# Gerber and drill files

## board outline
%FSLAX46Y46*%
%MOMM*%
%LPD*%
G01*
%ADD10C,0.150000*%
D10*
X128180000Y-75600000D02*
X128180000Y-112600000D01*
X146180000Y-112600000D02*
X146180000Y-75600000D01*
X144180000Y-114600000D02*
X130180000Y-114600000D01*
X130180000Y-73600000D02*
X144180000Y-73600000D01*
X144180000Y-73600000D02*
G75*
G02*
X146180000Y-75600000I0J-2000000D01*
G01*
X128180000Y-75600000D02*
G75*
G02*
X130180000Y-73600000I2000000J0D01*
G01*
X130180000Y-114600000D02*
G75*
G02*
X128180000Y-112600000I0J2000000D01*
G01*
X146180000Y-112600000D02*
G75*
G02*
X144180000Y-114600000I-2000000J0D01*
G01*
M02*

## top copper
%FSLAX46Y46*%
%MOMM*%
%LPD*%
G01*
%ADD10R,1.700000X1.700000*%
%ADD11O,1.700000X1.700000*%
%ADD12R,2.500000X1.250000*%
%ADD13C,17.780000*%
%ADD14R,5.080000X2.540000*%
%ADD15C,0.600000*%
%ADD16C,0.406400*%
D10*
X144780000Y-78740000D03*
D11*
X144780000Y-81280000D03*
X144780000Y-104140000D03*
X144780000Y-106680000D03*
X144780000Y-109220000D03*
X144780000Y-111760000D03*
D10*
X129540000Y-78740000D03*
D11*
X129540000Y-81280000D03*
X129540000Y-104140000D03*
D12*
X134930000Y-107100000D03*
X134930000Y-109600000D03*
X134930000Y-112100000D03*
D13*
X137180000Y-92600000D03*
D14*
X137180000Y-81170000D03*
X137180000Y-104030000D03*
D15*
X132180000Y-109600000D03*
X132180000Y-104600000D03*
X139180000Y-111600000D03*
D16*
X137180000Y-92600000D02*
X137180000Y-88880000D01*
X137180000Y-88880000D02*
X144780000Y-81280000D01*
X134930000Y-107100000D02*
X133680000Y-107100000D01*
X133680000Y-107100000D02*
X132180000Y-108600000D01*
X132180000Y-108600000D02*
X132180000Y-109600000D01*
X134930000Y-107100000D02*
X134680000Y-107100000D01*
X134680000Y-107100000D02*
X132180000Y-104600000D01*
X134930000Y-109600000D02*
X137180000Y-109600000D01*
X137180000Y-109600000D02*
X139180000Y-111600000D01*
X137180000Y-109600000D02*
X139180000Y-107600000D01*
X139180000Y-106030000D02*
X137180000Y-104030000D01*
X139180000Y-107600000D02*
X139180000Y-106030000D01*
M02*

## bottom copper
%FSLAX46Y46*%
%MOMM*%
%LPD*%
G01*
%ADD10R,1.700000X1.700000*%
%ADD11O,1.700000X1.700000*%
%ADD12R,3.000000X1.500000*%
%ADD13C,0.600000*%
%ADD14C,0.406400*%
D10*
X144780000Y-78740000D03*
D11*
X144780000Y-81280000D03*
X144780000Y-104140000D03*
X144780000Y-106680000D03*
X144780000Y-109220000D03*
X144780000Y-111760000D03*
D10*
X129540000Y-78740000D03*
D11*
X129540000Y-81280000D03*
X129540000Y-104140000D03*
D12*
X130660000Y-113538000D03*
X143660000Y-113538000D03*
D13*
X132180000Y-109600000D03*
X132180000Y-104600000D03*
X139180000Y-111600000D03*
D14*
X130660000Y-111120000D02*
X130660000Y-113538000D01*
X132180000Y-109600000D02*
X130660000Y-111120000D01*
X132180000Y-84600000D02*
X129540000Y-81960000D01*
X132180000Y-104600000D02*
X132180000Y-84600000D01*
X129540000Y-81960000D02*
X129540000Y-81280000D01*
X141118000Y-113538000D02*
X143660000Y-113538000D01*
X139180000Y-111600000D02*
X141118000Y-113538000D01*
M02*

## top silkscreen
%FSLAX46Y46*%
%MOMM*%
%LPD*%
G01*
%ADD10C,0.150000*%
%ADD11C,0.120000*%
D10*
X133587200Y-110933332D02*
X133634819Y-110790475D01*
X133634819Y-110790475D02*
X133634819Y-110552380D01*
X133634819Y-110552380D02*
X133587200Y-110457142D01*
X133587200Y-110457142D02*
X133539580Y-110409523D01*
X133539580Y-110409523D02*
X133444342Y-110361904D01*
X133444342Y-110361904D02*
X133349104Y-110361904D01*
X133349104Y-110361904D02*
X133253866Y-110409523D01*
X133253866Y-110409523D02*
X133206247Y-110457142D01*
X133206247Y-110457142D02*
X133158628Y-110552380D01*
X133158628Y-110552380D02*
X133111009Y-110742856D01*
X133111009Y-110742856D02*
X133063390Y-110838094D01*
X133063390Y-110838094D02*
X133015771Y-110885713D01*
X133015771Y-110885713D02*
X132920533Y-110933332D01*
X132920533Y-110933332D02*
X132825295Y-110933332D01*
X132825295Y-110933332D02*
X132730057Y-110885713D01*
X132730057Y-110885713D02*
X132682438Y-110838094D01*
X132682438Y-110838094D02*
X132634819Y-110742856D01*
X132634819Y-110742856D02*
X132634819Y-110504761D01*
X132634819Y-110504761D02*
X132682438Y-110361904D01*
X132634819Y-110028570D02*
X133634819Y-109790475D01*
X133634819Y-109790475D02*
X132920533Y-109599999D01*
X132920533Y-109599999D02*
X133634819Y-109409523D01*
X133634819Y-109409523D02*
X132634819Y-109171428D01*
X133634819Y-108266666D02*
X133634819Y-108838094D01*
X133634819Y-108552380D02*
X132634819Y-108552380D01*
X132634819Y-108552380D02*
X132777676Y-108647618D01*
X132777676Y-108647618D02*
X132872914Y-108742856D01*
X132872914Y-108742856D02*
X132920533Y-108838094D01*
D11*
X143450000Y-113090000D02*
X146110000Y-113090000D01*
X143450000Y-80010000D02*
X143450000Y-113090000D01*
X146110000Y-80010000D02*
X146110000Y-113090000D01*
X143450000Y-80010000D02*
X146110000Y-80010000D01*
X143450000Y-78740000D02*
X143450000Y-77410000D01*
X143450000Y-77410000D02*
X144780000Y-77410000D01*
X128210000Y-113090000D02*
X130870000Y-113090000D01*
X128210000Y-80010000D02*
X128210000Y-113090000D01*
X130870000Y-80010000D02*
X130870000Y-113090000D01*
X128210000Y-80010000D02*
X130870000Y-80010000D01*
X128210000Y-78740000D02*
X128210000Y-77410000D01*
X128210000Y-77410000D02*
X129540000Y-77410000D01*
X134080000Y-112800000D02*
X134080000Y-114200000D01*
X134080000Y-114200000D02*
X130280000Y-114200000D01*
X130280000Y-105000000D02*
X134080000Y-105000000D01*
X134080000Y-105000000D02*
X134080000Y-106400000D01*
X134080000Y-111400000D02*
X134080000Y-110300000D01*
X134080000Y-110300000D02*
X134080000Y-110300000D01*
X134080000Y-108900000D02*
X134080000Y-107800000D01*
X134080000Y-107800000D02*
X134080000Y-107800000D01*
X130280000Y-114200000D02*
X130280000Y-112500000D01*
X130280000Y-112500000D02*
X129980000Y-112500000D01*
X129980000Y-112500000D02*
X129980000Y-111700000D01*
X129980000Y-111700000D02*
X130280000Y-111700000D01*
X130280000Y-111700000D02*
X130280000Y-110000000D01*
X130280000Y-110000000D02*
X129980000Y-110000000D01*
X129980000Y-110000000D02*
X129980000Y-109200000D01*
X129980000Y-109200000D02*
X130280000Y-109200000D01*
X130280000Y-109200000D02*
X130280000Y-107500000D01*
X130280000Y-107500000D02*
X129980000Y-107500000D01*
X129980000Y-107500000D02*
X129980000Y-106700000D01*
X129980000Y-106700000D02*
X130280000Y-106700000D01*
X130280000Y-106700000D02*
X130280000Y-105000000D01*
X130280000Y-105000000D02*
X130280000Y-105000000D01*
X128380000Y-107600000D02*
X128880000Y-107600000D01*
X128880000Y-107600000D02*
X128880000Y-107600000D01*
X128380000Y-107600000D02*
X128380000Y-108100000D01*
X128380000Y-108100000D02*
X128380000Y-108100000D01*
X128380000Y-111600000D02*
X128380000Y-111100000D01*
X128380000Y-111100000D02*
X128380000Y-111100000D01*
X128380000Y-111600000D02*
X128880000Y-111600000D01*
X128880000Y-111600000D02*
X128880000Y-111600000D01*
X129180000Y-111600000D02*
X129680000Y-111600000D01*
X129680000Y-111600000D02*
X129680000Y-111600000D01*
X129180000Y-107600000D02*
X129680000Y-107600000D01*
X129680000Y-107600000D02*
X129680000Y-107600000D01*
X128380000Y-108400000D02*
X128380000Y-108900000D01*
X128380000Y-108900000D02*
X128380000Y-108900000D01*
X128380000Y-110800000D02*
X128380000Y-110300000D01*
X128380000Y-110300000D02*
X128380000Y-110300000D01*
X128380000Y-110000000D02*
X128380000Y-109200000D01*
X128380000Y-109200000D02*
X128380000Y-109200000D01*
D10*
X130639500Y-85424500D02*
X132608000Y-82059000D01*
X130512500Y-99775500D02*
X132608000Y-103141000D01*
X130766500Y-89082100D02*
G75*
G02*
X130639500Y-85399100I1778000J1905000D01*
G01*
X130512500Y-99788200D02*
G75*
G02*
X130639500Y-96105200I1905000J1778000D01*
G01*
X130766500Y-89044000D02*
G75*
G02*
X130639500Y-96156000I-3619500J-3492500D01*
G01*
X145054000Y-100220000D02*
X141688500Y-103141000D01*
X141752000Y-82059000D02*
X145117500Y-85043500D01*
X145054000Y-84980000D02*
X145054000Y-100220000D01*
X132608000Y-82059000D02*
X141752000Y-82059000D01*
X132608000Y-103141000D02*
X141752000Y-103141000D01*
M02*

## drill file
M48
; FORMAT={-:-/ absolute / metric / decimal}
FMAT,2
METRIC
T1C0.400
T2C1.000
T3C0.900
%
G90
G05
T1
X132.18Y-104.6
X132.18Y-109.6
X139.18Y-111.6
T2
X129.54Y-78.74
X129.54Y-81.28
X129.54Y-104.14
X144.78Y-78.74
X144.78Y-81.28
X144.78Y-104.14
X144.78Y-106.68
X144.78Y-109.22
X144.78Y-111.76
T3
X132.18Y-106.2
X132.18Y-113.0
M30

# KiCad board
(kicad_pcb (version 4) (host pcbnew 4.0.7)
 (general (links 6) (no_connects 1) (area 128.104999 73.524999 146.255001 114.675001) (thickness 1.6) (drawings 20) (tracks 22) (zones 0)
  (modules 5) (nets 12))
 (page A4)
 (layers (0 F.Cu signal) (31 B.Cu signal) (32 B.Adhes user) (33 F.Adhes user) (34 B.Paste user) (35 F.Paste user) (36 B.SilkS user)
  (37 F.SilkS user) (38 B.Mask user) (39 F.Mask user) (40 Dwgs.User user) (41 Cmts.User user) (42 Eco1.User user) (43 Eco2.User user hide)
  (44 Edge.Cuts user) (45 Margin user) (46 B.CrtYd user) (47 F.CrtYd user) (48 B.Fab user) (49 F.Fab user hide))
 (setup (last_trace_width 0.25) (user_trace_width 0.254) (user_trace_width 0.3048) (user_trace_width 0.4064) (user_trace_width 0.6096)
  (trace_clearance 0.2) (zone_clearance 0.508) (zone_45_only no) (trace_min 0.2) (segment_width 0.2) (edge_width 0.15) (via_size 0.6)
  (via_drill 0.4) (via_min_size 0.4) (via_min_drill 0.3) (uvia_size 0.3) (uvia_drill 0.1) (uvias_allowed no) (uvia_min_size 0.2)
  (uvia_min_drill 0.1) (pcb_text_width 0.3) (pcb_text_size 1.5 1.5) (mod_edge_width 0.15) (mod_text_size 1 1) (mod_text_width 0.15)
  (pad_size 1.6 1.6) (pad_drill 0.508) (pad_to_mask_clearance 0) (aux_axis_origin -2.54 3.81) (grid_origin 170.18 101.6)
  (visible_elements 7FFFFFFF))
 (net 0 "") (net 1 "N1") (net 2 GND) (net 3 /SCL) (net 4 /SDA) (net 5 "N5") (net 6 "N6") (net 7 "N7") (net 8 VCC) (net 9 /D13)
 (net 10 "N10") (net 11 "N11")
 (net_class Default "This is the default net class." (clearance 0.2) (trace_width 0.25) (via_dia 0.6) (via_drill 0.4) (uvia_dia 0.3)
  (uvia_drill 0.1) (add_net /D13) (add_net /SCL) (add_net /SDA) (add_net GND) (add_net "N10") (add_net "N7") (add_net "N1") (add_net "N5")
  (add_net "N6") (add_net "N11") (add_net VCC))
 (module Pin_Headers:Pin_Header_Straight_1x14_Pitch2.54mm (layer F.Cu) (at 144.78 78.74)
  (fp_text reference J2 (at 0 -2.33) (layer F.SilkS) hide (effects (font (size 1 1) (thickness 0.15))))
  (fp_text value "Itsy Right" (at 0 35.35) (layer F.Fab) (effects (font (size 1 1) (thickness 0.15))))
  (fp_line (start -1.33 34.35) (end 1.33 34.35) (layer F.SilkS) (width 0.12))
  (fp_line (start -1.33 1.27) (end -1.33 34.35) (layer F.SilkS) (width 0.12))
  (fp_line (start 1.33 1.27) (end 1.33 34.35) (layer F.SilkS) (width 0.12))
  (fp_line (start -1.33 1.27) (end 1.33 1.27) (layer F.SilkS) (width 0.12))
  (fp_line (start -1.33 0) (end -1.33 -1.33) (layer F.SilkS) (width 0.12))
  (fp_line (start -1.33 -1.33) (end 0 -1.33) (layer F.SilkS) (width 0.12))
  (pad 1 thru_hole rect (at 0 0) (size 1.7 1.7) (drill 1) (layers *.Cu *.Mask) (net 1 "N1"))
  (pad 2 thru_hole oval (at 0 2.54) (size 1.7 1.7) (drill 1) (layers *.Cu *.Mask) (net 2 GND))
  (pad 11 thru_hole oval (at 0 25.4) (size 1.7 1.7) (drill 1) (layers *.Cu *.Mask) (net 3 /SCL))
  (pad 12 thru_hole oval (at 0 27.94) (size 1.7 1.7) (drill 1) (layers *.Cu *.Mask) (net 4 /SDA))
  (pad 13 thru_hole oval (at 0 30.48) (size 1.7 1.7) (drill 1) (layers *.Cu *.Mask) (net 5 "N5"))
  (pad 14 thru_hole oval (at 0 33.02) (size 1.7 1.7) (drill 1) (layers *.Cu *.Mask) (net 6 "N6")))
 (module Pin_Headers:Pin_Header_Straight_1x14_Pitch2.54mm (layer F.Cu) (at 129.54 78.74)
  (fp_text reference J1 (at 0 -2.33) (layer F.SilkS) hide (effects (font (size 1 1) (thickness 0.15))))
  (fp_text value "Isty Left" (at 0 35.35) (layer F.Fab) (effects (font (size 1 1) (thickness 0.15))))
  (fp_line (start -1.33 34.35) (end 1.33 34.35) (layer F.SilkS) (width 0.12))
  (fp_line (start -1.33 1.27) (end -1.33 34.35) (layer F.SilkS) (width 0.12))
  (fp_line (start 1.33 1.27) (end 1.33 34.35) (layer F.SilkS) (width 0.12))
  (fp_line (start -1.33 1.27) (end 1.33 1.27) (layer F.SilkS) (width 0.12))
  (fp_line (start -1.33 0) (end -1.33 -1.33) (layer F.SilkS) (width 0.12))
  (fp_line (start -1.33 -1.33) (end 0 -1.33) (layer F.SilkS) (width 0.12))
  (pad 1 thru_hole rect (at 0 0) (size 1.7 1.7) (drill 1) (layers *.Cu *.Mask) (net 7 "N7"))
  (pad 2 thru_hole oval (at 0 2.54) (size 1.7 1.7) (drill 1) (layers *.Cu *.Mask) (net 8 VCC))
  (pad 11 thru_hole oval (at 0 25.4) (size 1.7 1.7) (drill 1) (layers *.Cu *.Mask) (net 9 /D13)))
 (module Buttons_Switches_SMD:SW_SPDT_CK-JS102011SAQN (layer F.Cu) (at 132.18 109.6 270)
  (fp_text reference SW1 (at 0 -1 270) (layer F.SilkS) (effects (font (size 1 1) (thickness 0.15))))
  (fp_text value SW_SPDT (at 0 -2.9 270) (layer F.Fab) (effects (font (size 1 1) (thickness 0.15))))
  (fp_line (start 3.2 -1.9) (end 4.6 -1.9) (layer F.SilkS) (width 0.12))
  (fp_line (start 4.6 -1.9) (end 4.6 1.9) (layer F.SilkS) (width 0.12))
  (fp_line (start -4.6 1.9) (end -4.6 -1.9) (layer F.SilkS) (width 0.12))
  (fp_line (start -4.6 -1.9) (end -3.2 -1.9) (layer F.SilkS) (width 0.12))
  (fp_line (start 1.8 -1.9) (end 0.7 -1.9) (layer F.SilkS) (width 0.12))
  (fp_line (start 0.7 -1.9) (end 0.7 -1.9) (layer F.SilkS) (width 0.12))
  (fp_line (start -0.7 -1.9) (end -1.8 -1.9) (layer F.SilkS) (width 0.12))
  (fp_line (start -1.8 -1.9) (end -1.8 -1.9) (layer F.SilkS) (width 0.12))
  (fp_line (start 4.6 1.9) (end 2.9 1.9) (layer F.SilkS) (width 0.12))
  (fp_line (start 2.9 1.9) (end 2.9 2.2) (layer F.SilkS) (width 0.12))
  (fp_line (start 2.9 2.2) (end 2.1 2.2) (layer F.SilkS) (width 0.12))
  (fp_line (start 2.1 2.2) (end 2.1 1.9) (layer F.SilkS) (width 0.12))
  (fp_line (start 2.1 1.9) (end 0.4 1.9) (layer F.SilkS) (width 0.12))
  (fp_line (start 0.4 1.9) (end 0.4 2.2) (layer F.SilkS) (width 0.12))
  (fp_line (start 0.4 2.2) (end -0.4 2.2) (layer F.SilkS) (width 0.12))
  (fp_line (start -0.4 2.2) (end -0.4 1.9) (layer F.SilkS) (width 0.12))
  (fp_line (start -0.4 1.9) (end -2.1 1.9) (layer F.SilkS) (width 0.12))
  (fp_line (start -2.1 1.9) (end -2.1 2.2) (layer F.SilkS) (width 0.12))
  (fp_line (start -2.1 2.2) (end -2.9 2.2) (layer F.SilkS) (width 0.12))
  (fp_line (start -2.9 2.2) (end -2.9 1.9) (layer F.SilkS) (width 0.12))
  (fp_line (start -2.9 1.9) (end -4.6 1.9) (layer F.SilkS) (width 0.12))
  (fp_line (start -4.6 1.9) (end -4.6 1.9) (layer F.SilkS) (width 0.12))
  (fp_line (start -2 3.8) (end -2 3.3) (layer F.SilkS) (width 0.12))
  (fp_line (start -2 3.3) (end -2 3.3) (layer F.SilkS) (width 0.12))
  (fp_line (start -2 3.8) (end -1.5 3.8) (layer F.SilkS) (width 0.12))
  (fp_line (start -1.5 3.8) (end -1.5 3.8) (layer F.SilkS) (width 0.12))
  (fp_line (start 2 3.8) (end 1.5 3.8) (layer F.SilkS) (width 0.12))
  (fp_line (start 1.5 3.8) (end 1.5 3.8) (layer F.SilkS) (width 0.12))
  (fp_line (start 2 3.8) (end 2 3.3) (layer F.SilkS) (width 0.12))
  (fp_line (start 2 3.3) (end 2 3.3) (layer F.SilkS) (width 0.12))
  (fp_line (start 2 3) (end 2 2.5) (layer F.SilkS) (width 0.12))
  (fp_line (start 2 2.5) (end 2 2.5) (layer F.SilkS) (width 0.12))
  (fp_line (start -2 3) (end -2 2.5) (layer F.SilkS) (width 0.12))
  (fp_line (start -2 2.5) (end -2 2.5) (layer F.SilkS) (width 0.12))
  (fp_line (start -1.2 3.8) (end -0.7 3.8) (layer F.SilkS) (width 0.12))
  (fp_line (start -0.7 3.8) (end -0.7 3.8) (layer F.SilkS) (width 0.12))
  (fp_line (start 1.2 3.8) (end 0.7 3.8) (layer F.SilkS) (width 0.12))
  (fp_line (start 0.7 3.8) (end 0.7 3.8) (layer F.SilkS) (width 0.12))
  (fp_line (start 0.4 3.8) (end -0.4 3.8) (layer F.SilkS) (width 0.12))
  (fp_line (start -0.4 3.8) (end -0.4 3.8) (layer F.SilkS) (width 0.12))
  (pad 1 smd rect (at -2.5 -2.75 270) (size 1.25 2.5) (layers F.Cu F.Paste F.Mask) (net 8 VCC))
  (pad 2 smd rect (at 0 -2.75 270) (size 1.25 2.5) (layers F.Cu F.Paste F.Mask) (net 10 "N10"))
  (pad 3 smd rect (at 2.5 -2.75 270) (size 1.25 2.5) (layers F.Cu F.Paste F.Mask) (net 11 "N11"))
  (pad "" np_thru_hole circle (at -3.4 0 270) (size 0.9 0.9) (drill 0.9) (layers *.Cu *.Mask))
  (pad "" np_thru_hole circle (at 3.4 0 270) (size 0.9 0.9) (drill 0.9) (layers *.Cu *.Mask)))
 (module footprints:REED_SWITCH (layer B.Cu) (at 137.16 113.538)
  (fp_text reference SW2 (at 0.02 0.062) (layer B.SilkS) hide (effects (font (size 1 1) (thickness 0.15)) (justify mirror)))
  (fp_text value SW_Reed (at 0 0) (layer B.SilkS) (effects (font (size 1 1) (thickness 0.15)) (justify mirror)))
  (pad 1 smd rect (at -6.5 0) (size 3 1.5) (layers B.Cu B.Paste B.Mask) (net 8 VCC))
  (pad 2 smd rect (at 6.5 0) (size 3 1.5) (layers B.Cu B.Paste B.Mask) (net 10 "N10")))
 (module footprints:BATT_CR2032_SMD (layer F.Cu) (at 137.18 92.6 270)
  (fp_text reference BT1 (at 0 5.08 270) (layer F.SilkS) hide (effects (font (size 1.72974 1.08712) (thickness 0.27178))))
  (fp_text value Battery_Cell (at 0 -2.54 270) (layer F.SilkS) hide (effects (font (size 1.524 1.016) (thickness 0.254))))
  (fp_line (start -7.1755 6.5405) (end -10.541 4.572) (layer F.SilkS) (width 0.15))
  (fp_line (start 7.1755 6.6675) (end 10.541 4.572) (layer F.SilkS) (width 0.15))
  (fp_arc (start -5.4229 4.6355) (end -3.5179 6.4135) (angle 90) (layer F.SilkS) (width 0.15))
  (fp_arc (start 5.4102 4.7625) (end 7.1882 6.6675) (angle 90) (layer F.SilkS) (width 0.15))
  (fp_arc (start -0.0635 10.033) (end -3.556 6.4135) (angle 90) (layer F.SilkS) (width 0.15))
  (fp_line (start 7.62 -7.874) (end 10.541 -4.5085) (layer F.SilkS) (width 0.15))
  (fp_line (start -10.541 -4.572) (end -7.5565 -7.9375) (layer F.SilkS) (width 0.15))
  (fp_line (start -7.62 -7.874) (end 7.62 -7.874) (layer F.SilkS) (width 0.15))
  (fp_line (start -10.541 4.572) (end -10.541 -4.572) (layer F.SilkS) (width 0.15))
  (fp_line (start 10.541 4.572) (end 10.541 -4.572) (layer F.SilkS) (width 0.15))
  (pad 2 smd circle (at 0 0 270) (size 17.78 17.78) (layers F.Cu F.Paste F.Mask) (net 2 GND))
  (pad 1 smd rect (at -11.43 0 270) (size 2.54 5.08) (layers F.Cu F.Paste F.Mask) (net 10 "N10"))
  (pad 1 smd rect (at 11.43 0 270) (size 2.54 5.08) (layers F.Cu F.Paste F.Mask) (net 10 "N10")))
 (gr_line (start 128.18 75.6) (end 128.18 112.6) (angle 90) (layer Edge.Cuts) (width 0.15))
 (gr_line (start 146.18 112.6) (end 146.18 75.6) (angle 90) (layer Edge.Cuts) (width 0.15))
 (gr_line (start 144.18 114.6) (end 130.18 114.6) (angle 90) (layer Edge.Cuts) (width 0.15))
 (gr_line (start 130.18 73.6) (end 144.18 73.6) (angle 90) (layer Edge.Cuts) (width 0.15))
 (gr_arc (start 144.18 75.6) (end 144.18 73.6) (angle 90) (layer Edge.Cuts) (width 0.15))
 (gr_arc (start 130.18 75.6) (end 128.18 75.6) (angle 90) (layer Edge.Cuts) (width 0.15))
 (gr_arc (start 130.18 112.6) (end 130.18 114.6) (angle 90) (layer Edge.Cuts) (width 0.15))
 (gr_arc (start 144.18 112.6) (end 146.18 112.6) (angle 90) (layer Edge.Cuts) (width 0.15))
 (segment (start 137.18 92.6) (end 137.18 88.88) (width 0.4064) (layer F.Cu) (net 2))
 (segment (start 137.18 88.88) (end 144.78 81.28) (width 0.4064) (layer F.Cu) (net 2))
 (segment (start 134.93 107.1) (end 133.68 107.1) (width 0.4064) (layer F.Cu) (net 8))
 (segment (start 133.68 107.1) (end 132.18 108.6) (width 0.4064) (layer F.Cu) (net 8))
 (segment (start 130.66 111.12) (end 130.66 113.538) (width 0.4064) (layer B.Cu) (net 8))
 (segment (start 132.18 109.6) (end 130.66 111.12) (width 0.4064) (layer B.Cu) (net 8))
 (via (at 132.18 109.6) (size 0.6) (drill 0.4) (layers F.Cu B.Cu) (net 8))
 (segment (start 132.18 108.6) (end 132.18 109.6) (width 0.4064) (layer F.Cu) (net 8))
 (segment (start 134.93 107.1) (end 134.68 107.1) (width 0.4064) (layer F.Cu) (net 8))
 (segment (start 134.68 107.1) (end 132.18 104.6) (width 0.4064) (layer F.Cu) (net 8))
 (segment (start 132.18 84.6) (end 129.54 81.96) (width 0.4064) (layer B.Cu) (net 8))
 (segment (start 132.18 104.6) (end 132.18 84.6) (width 0.4064) (layer B.Cu) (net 8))
 (via (at 132.18 104.6) (size 0.6) (drill 0.4) (layers F.Cu B.Cu) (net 8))
 (segment (start 129.54 81.96) (end 129.54 81.28) (width 0.4064) (layer B.Cu) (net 8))
 (segment (start 134.93 109.6) (end 137.18 109.6) (width 0.4064) (layer F.Cu) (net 10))
 (segment (start 137.18 109.6) (end 139.18 111.6) (width 0.4064) (layer F.Cu) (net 10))
 (segment (start 141.118 113.538) (end 143.66 113.538) (width 0.4064) (layer B.Cu) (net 10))
 (segment (start 139.18 111.6) (end 141.118 113.538) (width 0.4064) (layer B.Cu) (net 10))
 (via (at 139.18 111.6) (size 0.6) (drill 0.4) (layers F.Cu B.Cu) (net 10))
 (segment (start 137.18 109.6) (end 139.18 107.6) (width 0.4064) (layer F.Cu) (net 10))
 (segment (start 139.18 106.03) (end 137.18 104.03) (width 0.4064) (layer F.Cu) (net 10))
 (segment (start 139.18 107.6) (end 139.18 106.03) (width 0.4064) (layer F.Cu) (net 10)))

